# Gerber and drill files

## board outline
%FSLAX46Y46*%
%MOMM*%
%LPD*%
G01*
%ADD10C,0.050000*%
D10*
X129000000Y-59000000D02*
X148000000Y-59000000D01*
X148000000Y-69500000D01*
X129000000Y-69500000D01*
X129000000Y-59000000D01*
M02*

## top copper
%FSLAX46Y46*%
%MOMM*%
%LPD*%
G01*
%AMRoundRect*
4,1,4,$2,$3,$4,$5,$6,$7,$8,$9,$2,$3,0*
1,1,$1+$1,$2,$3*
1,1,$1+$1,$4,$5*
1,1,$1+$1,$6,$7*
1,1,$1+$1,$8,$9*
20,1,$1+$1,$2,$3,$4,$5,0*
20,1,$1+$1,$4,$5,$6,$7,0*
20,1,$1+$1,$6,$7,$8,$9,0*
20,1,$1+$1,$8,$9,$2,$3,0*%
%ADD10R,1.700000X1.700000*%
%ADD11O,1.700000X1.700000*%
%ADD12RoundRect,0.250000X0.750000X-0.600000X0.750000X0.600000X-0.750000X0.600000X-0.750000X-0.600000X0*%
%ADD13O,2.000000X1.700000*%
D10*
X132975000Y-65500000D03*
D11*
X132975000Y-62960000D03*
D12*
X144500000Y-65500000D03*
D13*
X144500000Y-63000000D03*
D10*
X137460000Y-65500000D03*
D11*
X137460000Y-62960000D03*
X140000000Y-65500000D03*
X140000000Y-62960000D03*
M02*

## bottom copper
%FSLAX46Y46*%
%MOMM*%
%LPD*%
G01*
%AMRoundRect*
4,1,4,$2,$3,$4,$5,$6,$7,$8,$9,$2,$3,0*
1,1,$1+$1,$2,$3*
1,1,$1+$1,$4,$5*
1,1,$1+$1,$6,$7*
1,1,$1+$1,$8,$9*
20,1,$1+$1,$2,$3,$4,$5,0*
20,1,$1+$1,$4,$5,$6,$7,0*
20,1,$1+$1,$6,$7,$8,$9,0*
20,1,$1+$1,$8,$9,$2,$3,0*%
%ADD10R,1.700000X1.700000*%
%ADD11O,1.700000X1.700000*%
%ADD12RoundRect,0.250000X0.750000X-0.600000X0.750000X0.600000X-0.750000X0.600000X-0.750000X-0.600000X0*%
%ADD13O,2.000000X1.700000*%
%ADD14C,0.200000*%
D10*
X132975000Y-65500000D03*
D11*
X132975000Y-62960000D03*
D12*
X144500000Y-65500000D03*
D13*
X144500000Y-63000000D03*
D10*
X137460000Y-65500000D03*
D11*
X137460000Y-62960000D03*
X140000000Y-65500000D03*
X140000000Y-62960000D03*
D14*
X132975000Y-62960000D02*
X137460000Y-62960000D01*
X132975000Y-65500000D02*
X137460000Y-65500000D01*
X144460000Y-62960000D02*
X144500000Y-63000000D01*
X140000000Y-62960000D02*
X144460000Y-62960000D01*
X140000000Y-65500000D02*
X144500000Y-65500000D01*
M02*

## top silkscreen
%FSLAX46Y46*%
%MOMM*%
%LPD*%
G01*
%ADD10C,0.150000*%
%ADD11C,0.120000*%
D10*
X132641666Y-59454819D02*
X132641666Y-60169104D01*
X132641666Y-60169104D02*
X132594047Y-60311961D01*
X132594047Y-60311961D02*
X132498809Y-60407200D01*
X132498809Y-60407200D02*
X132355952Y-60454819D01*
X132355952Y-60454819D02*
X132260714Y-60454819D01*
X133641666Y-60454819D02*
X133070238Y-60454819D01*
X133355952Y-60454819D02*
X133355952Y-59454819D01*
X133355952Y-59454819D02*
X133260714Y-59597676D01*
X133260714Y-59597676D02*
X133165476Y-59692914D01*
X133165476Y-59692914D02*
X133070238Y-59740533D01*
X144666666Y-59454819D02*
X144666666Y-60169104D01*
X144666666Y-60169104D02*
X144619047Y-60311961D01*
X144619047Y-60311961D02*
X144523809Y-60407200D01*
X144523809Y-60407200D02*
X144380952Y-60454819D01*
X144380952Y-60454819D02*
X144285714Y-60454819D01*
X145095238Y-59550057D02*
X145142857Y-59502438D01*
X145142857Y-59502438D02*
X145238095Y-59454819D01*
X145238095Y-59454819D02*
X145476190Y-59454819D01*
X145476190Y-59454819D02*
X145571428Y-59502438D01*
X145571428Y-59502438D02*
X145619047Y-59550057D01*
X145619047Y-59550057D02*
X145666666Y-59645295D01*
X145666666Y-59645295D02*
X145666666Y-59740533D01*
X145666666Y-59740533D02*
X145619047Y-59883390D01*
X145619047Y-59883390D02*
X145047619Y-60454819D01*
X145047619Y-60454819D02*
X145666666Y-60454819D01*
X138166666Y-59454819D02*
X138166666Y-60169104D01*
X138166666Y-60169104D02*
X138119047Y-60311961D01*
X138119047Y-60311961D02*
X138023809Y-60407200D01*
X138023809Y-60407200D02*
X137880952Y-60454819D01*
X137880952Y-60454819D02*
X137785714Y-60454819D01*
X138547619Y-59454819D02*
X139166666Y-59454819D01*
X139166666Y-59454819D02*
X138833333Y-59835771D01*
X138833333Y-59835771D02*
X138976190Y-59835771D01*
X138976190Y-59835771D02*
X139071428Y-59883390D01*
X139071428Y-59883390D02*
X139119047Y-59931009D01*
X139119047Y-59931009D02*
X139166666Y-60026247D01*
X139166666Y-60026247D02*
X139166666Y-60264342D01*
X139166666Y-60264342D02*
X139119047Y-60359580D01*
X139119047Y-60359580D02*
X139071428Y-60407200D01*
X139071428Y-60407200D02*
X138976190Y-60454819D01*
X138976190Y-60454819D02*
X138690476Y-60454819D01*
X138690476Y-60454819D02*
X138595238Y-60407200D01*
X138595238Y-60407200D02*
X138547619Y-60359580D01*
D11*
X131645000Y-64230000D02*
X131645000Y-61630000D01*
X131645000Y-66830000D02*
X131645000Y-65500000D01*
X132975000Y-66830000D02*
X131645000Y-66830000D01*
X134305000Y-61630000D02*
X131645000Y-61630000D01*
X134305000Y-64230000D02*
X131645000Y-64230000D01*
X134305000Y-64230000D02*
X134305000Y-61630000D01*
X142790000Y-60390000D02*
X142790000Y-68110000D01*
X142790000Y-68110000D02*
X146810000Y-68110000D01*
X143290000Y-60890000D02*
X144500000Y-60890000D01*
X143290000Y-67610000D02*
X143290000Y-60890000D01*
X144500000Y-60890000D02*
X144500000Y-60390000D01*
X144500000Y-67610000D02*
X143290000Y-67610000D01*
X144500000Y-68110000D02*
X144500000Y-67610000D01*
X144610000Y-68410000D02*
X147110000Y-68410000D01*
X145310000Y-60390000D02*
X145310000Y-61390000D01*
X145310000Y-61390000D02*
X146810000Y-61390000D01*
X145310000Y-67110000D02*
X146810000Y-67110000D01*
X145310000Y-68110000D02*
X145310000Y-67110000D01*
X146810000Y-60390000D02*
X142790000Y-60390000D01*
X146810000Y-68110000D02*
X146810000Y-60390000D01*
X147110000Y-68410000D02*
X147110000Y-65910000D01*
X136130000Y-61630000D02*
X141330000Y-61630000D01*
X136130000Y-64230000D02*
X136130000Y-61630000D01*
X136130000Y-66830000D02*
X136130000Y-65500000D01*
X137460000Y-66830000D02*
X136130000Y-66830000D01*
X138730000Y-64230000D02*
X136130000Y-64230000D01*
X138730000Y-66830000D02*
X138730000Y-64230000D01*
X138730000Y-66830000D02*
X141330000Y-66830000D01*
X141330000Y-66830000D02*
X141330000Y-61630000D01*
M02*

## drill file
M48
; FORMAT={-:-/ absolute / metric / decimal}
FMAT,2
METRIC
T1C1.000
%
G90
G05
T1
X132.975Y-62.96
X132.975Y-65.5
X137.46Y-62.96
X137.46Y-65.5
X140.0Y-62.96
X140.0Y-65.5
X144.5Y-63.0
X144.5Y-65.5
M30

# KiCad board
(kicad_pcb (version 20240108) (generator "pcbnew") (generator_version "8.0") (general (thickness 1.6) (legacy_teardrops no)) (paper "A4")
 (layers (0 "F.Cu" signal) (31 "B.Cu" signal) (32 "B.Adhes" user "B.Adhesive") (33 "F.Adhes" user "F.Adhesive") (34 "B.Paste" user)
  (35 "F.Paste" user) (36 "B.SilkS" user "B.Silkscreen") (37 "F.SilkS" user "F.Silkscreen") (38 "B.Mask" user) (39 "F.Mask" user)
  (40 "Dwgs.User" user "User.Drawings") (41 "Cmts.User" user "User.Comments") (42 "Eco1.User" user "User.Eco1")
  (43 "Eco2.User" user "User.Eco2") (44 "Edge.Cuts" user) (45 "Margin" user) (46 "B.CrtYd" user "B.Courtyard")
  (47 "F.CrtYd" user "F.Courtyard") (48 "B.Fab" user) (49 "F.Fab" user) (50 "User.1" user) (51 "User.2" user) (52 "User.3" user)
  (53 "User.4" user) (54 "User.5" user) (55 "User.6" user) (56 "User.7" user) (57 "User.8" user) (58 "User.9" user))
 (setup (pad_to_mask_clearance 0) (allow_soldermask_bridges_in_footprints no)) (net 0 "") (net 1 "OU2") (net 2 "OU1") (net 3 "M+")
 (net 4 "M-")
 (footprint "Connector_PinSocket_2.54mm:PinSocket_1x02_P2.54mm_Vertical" (layer "F.Cu") (at 132.975 65.5 180)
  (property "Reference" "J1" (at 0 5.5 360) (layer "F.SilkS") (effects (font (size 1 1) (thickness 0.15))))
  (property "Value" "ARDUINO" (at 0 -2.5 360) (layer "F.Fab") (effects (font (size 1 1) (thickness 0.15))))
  (fp_line (start 1.33 1.27) (end 1.33 3.87) (stroke (width 0.12) (type solid)) (layer "F.SilkS"))
  (fp_line (start 1.33 -1.33) (end 1.33 0) (stroke (width 0.12) (type solid)) (layer "F.SilkS"))
  (fp_line (start 0 -1.33) (end 1.33 -1.33) (stroke (width 0.12) (type solid)) (layer "F.SilkS"))
  (fp_line (start -1.33 3.87) (end 1.33 3.87) (stroke (width 0.12) (type solid)) (layer "F.SilkS"))
  (fp_line (start -1.33 1.27) (end 1.33 1.27) (stroke (width 0.12) (type solid)) (layer "F.SilkS"))
  (fp_line (start -1.33 1.27) (end -1.33 3.87) (stroke (width 0.12) (type solid)) (layer "F.SilkS"))
  (pad "1" thru_hole rect (at 0 0 180) (size 1.7 1.7) (drill 1) (layers "*.Cu" "*.Mask") (remove_unused_layers no) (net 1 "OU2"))
  (pad "2" thru_hole oval (at 0 2.54 180) (size 1.7 1.7) (drill 1) (layers "*.Cu" "*.Mask") (remove_unused_layers no) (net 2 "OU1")))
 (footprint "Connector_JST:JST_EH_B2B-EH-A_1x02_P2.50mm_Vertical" (layer "F.Cu") (at 144.5 65.5 90)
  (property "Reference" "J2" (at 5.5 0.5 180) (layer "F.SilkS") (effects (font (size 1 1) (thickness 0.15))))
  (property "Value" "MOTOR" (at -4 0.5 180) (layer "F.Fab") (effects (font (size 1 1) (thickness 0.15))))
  (fp_line (start 5.11 -1.71) (end -2.61 -1.71) (stroke (width 0.12) (type solid)) (layer "F.SilkS"))
  (fp_line (start -2.61 -1.71) (end -2.61 2.31) (stroke (width 0.12) (type solid)) (layer "F.SilkS"))
  (fp_line (start 4.61 -1.21) (end 4.61 0) (stroke (width 0.12) (type solid)) (layer "F.SilkS"))
  (fp_line (start -2.11 -1.21) (end 4.61 -1.21) (stroke (width 0.12) (type solid)) (layer "F.SilkS"))
  (fp_line (start 4.61 0) (end 5.11 0) (stroke (width 0.12) (type solid)) (layer "F.SilkS"))
  (fp_line (start -2.11 0) (end -2.11 -1.21) (stroke (width 0.12) (type solid)) (layer "F.SilkS"))
  (fp_line (start -2.61 0) (end -2.11 0) (stroke (width 0.12) (type solid)) (layer "F.SilkS"))
  (fp_line (start -2.91 0.11) (end -2.91 2.61) (stroke (width 0.12) (type solid)) (layer "F.SilkS"))
  (fp_line (start 5.11 0.81) (end 4.11 0.81) (stroke (width 0.12) (type solid)) (layer "F.SilkS"))
  (fp_line (start 4.11 0.81) (end 4.11 2.31) (stroke (width 0.12) (type solid)) (layer "F.SilkS"))
  (fp_line (start -1.61 0.81) (end -1.61 2.31) (stroke (width 0.12) (type solid)) (layer "F.SilkS"))
  (fp_line (start -2.61 0.81) (end -1.61 0.81) (stroke (width 0.12) (type solid)) (layer "F.SilkS"))
  (fp_line (start 5.11 2.31) (end 5.11 -1.71) (stroke (width 0.12) (type solid)) (layer "F.SilkS"))
  (fp_line (start -2.61 2.31) (end 5.11 2.31) (stroke (width 0.12) (type solid)) (layer "F.SilkS"))
  (fp_line (start -2.91 2.61) (end -0.41 2.61) (stroke (width 0.12) (type solid)) (layer "F.SilkS"))
  (pad "1" thru_hole roundrect (at 0 0 90) (size 1.7 2) (drill 1) (layers "*.Cu" "*.Mask") (remove_unused_layers no)
   (roundrect_rratio 0.147059) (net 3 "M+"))
  (pad "2" thru_hole oval (at 2.5 0 90) (size 1.7 2) (drill 1) (layers "*.Cu" "*.Mask") (remove_unused_layers no) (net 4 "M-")))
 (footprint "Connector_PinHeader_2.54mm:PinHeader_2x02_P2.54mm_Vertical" (layer "F.Cu") (at 137.46 65.5 90)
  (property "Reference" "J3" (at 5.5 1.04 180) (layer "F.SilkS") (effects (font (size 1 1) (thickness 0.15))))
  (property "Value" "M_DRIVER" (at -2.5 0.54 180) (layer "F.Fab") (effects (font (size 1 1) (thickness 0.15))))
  (fp_line (start 3.87 -1.33) (end 3.87 3.87) (stroke (width 0.12) (type solid)) (layer "F.SilkS"))
  (fp_line (start 1.27 -1.33) (end 3.87 -1.33) (stroke (width 0.12) (type solid)) (layer "F.SilkS"))
  (fp_line (start -1.33 -1.33) (end 0 -1.33) (stroke (width 0.12) (type solid)) (layer "F.SilkS"))
  (fp_line (start -1.33 0) (end -1.33 -1.33) (stroke (width 0.12) (type solid)) (layer "F.SilkS"))
  (fp_line (start 1.27 1.27) (end 1.27 -1.33) (stroke (width 0.12) (type solid)) (layer "F.SilkS"))
  (fp_line (start -1.33 1.27) (end 1.27 1.27) (stroke (width 0.12) (type solid)) (layer "F.SilkS"))
  (fp_line (start -1.33 1.27) (end -1.33 3.87) (stroke (width 0.12) (type solid)) (layer "F.SilkS"))
  (fp_line (start -1.33 3.87) (end 3.87 3.87) (stroke (width 0.12) (type solid)) (layer "F.SilkS"))
  (pad "1" thru_hole rect (at 0 0 90) (size 1.7 1.7) (drill 1) (layers "*.Cu" "*.Mask") (remove_unused_layers no) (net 1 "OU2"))
  (pad "2" thru_hole oval (at 2.54 0 90) (size 1.7 1.7) (drill 1) (layers "*.Cu" "*.Mask") (remove_unused_layers no) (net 2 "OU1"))
  (pad "3" thru_hole oval (at 0 2.54 90) (size 1.7 1.7) (drill 1) (layers "*.Cu" "*.Mask") (remove_unused_layers no) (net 3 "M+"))
  (pad "4" thru_hole oval (at 2.54 2.54 90) (size 1.7 1.7) (drill 1) (layers "*.Cu" "*.Mask") (remove_unused_layers no) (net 4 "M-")))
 (gr_rect (start 129 59) (end 148 69.5) (stroke (width 0.05) (type default)) (fill none) (layer "Edge.Cuts"))
 (segment (start 132.975 62.96) (end 137.46 62.96) (width 0.2) (layer "B.Cu") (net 2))
 (segment (start 132.975 65.5) (end 137.46 65.5) (width 0.2) (layer "B.Cu") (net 1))
 (segment (start 144.46 62.96) (end 144.5 63) (width 0.2) (layer "B.Cu") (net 4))
 (segment (start 140 62.96) (end 144.46 62.96) (width 0.2) (layer "B.Cu") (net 4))
 (segment (start 140 65.5) (end 144.5 65.5) (width 0.2) (layer "B.Cu") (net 3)))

